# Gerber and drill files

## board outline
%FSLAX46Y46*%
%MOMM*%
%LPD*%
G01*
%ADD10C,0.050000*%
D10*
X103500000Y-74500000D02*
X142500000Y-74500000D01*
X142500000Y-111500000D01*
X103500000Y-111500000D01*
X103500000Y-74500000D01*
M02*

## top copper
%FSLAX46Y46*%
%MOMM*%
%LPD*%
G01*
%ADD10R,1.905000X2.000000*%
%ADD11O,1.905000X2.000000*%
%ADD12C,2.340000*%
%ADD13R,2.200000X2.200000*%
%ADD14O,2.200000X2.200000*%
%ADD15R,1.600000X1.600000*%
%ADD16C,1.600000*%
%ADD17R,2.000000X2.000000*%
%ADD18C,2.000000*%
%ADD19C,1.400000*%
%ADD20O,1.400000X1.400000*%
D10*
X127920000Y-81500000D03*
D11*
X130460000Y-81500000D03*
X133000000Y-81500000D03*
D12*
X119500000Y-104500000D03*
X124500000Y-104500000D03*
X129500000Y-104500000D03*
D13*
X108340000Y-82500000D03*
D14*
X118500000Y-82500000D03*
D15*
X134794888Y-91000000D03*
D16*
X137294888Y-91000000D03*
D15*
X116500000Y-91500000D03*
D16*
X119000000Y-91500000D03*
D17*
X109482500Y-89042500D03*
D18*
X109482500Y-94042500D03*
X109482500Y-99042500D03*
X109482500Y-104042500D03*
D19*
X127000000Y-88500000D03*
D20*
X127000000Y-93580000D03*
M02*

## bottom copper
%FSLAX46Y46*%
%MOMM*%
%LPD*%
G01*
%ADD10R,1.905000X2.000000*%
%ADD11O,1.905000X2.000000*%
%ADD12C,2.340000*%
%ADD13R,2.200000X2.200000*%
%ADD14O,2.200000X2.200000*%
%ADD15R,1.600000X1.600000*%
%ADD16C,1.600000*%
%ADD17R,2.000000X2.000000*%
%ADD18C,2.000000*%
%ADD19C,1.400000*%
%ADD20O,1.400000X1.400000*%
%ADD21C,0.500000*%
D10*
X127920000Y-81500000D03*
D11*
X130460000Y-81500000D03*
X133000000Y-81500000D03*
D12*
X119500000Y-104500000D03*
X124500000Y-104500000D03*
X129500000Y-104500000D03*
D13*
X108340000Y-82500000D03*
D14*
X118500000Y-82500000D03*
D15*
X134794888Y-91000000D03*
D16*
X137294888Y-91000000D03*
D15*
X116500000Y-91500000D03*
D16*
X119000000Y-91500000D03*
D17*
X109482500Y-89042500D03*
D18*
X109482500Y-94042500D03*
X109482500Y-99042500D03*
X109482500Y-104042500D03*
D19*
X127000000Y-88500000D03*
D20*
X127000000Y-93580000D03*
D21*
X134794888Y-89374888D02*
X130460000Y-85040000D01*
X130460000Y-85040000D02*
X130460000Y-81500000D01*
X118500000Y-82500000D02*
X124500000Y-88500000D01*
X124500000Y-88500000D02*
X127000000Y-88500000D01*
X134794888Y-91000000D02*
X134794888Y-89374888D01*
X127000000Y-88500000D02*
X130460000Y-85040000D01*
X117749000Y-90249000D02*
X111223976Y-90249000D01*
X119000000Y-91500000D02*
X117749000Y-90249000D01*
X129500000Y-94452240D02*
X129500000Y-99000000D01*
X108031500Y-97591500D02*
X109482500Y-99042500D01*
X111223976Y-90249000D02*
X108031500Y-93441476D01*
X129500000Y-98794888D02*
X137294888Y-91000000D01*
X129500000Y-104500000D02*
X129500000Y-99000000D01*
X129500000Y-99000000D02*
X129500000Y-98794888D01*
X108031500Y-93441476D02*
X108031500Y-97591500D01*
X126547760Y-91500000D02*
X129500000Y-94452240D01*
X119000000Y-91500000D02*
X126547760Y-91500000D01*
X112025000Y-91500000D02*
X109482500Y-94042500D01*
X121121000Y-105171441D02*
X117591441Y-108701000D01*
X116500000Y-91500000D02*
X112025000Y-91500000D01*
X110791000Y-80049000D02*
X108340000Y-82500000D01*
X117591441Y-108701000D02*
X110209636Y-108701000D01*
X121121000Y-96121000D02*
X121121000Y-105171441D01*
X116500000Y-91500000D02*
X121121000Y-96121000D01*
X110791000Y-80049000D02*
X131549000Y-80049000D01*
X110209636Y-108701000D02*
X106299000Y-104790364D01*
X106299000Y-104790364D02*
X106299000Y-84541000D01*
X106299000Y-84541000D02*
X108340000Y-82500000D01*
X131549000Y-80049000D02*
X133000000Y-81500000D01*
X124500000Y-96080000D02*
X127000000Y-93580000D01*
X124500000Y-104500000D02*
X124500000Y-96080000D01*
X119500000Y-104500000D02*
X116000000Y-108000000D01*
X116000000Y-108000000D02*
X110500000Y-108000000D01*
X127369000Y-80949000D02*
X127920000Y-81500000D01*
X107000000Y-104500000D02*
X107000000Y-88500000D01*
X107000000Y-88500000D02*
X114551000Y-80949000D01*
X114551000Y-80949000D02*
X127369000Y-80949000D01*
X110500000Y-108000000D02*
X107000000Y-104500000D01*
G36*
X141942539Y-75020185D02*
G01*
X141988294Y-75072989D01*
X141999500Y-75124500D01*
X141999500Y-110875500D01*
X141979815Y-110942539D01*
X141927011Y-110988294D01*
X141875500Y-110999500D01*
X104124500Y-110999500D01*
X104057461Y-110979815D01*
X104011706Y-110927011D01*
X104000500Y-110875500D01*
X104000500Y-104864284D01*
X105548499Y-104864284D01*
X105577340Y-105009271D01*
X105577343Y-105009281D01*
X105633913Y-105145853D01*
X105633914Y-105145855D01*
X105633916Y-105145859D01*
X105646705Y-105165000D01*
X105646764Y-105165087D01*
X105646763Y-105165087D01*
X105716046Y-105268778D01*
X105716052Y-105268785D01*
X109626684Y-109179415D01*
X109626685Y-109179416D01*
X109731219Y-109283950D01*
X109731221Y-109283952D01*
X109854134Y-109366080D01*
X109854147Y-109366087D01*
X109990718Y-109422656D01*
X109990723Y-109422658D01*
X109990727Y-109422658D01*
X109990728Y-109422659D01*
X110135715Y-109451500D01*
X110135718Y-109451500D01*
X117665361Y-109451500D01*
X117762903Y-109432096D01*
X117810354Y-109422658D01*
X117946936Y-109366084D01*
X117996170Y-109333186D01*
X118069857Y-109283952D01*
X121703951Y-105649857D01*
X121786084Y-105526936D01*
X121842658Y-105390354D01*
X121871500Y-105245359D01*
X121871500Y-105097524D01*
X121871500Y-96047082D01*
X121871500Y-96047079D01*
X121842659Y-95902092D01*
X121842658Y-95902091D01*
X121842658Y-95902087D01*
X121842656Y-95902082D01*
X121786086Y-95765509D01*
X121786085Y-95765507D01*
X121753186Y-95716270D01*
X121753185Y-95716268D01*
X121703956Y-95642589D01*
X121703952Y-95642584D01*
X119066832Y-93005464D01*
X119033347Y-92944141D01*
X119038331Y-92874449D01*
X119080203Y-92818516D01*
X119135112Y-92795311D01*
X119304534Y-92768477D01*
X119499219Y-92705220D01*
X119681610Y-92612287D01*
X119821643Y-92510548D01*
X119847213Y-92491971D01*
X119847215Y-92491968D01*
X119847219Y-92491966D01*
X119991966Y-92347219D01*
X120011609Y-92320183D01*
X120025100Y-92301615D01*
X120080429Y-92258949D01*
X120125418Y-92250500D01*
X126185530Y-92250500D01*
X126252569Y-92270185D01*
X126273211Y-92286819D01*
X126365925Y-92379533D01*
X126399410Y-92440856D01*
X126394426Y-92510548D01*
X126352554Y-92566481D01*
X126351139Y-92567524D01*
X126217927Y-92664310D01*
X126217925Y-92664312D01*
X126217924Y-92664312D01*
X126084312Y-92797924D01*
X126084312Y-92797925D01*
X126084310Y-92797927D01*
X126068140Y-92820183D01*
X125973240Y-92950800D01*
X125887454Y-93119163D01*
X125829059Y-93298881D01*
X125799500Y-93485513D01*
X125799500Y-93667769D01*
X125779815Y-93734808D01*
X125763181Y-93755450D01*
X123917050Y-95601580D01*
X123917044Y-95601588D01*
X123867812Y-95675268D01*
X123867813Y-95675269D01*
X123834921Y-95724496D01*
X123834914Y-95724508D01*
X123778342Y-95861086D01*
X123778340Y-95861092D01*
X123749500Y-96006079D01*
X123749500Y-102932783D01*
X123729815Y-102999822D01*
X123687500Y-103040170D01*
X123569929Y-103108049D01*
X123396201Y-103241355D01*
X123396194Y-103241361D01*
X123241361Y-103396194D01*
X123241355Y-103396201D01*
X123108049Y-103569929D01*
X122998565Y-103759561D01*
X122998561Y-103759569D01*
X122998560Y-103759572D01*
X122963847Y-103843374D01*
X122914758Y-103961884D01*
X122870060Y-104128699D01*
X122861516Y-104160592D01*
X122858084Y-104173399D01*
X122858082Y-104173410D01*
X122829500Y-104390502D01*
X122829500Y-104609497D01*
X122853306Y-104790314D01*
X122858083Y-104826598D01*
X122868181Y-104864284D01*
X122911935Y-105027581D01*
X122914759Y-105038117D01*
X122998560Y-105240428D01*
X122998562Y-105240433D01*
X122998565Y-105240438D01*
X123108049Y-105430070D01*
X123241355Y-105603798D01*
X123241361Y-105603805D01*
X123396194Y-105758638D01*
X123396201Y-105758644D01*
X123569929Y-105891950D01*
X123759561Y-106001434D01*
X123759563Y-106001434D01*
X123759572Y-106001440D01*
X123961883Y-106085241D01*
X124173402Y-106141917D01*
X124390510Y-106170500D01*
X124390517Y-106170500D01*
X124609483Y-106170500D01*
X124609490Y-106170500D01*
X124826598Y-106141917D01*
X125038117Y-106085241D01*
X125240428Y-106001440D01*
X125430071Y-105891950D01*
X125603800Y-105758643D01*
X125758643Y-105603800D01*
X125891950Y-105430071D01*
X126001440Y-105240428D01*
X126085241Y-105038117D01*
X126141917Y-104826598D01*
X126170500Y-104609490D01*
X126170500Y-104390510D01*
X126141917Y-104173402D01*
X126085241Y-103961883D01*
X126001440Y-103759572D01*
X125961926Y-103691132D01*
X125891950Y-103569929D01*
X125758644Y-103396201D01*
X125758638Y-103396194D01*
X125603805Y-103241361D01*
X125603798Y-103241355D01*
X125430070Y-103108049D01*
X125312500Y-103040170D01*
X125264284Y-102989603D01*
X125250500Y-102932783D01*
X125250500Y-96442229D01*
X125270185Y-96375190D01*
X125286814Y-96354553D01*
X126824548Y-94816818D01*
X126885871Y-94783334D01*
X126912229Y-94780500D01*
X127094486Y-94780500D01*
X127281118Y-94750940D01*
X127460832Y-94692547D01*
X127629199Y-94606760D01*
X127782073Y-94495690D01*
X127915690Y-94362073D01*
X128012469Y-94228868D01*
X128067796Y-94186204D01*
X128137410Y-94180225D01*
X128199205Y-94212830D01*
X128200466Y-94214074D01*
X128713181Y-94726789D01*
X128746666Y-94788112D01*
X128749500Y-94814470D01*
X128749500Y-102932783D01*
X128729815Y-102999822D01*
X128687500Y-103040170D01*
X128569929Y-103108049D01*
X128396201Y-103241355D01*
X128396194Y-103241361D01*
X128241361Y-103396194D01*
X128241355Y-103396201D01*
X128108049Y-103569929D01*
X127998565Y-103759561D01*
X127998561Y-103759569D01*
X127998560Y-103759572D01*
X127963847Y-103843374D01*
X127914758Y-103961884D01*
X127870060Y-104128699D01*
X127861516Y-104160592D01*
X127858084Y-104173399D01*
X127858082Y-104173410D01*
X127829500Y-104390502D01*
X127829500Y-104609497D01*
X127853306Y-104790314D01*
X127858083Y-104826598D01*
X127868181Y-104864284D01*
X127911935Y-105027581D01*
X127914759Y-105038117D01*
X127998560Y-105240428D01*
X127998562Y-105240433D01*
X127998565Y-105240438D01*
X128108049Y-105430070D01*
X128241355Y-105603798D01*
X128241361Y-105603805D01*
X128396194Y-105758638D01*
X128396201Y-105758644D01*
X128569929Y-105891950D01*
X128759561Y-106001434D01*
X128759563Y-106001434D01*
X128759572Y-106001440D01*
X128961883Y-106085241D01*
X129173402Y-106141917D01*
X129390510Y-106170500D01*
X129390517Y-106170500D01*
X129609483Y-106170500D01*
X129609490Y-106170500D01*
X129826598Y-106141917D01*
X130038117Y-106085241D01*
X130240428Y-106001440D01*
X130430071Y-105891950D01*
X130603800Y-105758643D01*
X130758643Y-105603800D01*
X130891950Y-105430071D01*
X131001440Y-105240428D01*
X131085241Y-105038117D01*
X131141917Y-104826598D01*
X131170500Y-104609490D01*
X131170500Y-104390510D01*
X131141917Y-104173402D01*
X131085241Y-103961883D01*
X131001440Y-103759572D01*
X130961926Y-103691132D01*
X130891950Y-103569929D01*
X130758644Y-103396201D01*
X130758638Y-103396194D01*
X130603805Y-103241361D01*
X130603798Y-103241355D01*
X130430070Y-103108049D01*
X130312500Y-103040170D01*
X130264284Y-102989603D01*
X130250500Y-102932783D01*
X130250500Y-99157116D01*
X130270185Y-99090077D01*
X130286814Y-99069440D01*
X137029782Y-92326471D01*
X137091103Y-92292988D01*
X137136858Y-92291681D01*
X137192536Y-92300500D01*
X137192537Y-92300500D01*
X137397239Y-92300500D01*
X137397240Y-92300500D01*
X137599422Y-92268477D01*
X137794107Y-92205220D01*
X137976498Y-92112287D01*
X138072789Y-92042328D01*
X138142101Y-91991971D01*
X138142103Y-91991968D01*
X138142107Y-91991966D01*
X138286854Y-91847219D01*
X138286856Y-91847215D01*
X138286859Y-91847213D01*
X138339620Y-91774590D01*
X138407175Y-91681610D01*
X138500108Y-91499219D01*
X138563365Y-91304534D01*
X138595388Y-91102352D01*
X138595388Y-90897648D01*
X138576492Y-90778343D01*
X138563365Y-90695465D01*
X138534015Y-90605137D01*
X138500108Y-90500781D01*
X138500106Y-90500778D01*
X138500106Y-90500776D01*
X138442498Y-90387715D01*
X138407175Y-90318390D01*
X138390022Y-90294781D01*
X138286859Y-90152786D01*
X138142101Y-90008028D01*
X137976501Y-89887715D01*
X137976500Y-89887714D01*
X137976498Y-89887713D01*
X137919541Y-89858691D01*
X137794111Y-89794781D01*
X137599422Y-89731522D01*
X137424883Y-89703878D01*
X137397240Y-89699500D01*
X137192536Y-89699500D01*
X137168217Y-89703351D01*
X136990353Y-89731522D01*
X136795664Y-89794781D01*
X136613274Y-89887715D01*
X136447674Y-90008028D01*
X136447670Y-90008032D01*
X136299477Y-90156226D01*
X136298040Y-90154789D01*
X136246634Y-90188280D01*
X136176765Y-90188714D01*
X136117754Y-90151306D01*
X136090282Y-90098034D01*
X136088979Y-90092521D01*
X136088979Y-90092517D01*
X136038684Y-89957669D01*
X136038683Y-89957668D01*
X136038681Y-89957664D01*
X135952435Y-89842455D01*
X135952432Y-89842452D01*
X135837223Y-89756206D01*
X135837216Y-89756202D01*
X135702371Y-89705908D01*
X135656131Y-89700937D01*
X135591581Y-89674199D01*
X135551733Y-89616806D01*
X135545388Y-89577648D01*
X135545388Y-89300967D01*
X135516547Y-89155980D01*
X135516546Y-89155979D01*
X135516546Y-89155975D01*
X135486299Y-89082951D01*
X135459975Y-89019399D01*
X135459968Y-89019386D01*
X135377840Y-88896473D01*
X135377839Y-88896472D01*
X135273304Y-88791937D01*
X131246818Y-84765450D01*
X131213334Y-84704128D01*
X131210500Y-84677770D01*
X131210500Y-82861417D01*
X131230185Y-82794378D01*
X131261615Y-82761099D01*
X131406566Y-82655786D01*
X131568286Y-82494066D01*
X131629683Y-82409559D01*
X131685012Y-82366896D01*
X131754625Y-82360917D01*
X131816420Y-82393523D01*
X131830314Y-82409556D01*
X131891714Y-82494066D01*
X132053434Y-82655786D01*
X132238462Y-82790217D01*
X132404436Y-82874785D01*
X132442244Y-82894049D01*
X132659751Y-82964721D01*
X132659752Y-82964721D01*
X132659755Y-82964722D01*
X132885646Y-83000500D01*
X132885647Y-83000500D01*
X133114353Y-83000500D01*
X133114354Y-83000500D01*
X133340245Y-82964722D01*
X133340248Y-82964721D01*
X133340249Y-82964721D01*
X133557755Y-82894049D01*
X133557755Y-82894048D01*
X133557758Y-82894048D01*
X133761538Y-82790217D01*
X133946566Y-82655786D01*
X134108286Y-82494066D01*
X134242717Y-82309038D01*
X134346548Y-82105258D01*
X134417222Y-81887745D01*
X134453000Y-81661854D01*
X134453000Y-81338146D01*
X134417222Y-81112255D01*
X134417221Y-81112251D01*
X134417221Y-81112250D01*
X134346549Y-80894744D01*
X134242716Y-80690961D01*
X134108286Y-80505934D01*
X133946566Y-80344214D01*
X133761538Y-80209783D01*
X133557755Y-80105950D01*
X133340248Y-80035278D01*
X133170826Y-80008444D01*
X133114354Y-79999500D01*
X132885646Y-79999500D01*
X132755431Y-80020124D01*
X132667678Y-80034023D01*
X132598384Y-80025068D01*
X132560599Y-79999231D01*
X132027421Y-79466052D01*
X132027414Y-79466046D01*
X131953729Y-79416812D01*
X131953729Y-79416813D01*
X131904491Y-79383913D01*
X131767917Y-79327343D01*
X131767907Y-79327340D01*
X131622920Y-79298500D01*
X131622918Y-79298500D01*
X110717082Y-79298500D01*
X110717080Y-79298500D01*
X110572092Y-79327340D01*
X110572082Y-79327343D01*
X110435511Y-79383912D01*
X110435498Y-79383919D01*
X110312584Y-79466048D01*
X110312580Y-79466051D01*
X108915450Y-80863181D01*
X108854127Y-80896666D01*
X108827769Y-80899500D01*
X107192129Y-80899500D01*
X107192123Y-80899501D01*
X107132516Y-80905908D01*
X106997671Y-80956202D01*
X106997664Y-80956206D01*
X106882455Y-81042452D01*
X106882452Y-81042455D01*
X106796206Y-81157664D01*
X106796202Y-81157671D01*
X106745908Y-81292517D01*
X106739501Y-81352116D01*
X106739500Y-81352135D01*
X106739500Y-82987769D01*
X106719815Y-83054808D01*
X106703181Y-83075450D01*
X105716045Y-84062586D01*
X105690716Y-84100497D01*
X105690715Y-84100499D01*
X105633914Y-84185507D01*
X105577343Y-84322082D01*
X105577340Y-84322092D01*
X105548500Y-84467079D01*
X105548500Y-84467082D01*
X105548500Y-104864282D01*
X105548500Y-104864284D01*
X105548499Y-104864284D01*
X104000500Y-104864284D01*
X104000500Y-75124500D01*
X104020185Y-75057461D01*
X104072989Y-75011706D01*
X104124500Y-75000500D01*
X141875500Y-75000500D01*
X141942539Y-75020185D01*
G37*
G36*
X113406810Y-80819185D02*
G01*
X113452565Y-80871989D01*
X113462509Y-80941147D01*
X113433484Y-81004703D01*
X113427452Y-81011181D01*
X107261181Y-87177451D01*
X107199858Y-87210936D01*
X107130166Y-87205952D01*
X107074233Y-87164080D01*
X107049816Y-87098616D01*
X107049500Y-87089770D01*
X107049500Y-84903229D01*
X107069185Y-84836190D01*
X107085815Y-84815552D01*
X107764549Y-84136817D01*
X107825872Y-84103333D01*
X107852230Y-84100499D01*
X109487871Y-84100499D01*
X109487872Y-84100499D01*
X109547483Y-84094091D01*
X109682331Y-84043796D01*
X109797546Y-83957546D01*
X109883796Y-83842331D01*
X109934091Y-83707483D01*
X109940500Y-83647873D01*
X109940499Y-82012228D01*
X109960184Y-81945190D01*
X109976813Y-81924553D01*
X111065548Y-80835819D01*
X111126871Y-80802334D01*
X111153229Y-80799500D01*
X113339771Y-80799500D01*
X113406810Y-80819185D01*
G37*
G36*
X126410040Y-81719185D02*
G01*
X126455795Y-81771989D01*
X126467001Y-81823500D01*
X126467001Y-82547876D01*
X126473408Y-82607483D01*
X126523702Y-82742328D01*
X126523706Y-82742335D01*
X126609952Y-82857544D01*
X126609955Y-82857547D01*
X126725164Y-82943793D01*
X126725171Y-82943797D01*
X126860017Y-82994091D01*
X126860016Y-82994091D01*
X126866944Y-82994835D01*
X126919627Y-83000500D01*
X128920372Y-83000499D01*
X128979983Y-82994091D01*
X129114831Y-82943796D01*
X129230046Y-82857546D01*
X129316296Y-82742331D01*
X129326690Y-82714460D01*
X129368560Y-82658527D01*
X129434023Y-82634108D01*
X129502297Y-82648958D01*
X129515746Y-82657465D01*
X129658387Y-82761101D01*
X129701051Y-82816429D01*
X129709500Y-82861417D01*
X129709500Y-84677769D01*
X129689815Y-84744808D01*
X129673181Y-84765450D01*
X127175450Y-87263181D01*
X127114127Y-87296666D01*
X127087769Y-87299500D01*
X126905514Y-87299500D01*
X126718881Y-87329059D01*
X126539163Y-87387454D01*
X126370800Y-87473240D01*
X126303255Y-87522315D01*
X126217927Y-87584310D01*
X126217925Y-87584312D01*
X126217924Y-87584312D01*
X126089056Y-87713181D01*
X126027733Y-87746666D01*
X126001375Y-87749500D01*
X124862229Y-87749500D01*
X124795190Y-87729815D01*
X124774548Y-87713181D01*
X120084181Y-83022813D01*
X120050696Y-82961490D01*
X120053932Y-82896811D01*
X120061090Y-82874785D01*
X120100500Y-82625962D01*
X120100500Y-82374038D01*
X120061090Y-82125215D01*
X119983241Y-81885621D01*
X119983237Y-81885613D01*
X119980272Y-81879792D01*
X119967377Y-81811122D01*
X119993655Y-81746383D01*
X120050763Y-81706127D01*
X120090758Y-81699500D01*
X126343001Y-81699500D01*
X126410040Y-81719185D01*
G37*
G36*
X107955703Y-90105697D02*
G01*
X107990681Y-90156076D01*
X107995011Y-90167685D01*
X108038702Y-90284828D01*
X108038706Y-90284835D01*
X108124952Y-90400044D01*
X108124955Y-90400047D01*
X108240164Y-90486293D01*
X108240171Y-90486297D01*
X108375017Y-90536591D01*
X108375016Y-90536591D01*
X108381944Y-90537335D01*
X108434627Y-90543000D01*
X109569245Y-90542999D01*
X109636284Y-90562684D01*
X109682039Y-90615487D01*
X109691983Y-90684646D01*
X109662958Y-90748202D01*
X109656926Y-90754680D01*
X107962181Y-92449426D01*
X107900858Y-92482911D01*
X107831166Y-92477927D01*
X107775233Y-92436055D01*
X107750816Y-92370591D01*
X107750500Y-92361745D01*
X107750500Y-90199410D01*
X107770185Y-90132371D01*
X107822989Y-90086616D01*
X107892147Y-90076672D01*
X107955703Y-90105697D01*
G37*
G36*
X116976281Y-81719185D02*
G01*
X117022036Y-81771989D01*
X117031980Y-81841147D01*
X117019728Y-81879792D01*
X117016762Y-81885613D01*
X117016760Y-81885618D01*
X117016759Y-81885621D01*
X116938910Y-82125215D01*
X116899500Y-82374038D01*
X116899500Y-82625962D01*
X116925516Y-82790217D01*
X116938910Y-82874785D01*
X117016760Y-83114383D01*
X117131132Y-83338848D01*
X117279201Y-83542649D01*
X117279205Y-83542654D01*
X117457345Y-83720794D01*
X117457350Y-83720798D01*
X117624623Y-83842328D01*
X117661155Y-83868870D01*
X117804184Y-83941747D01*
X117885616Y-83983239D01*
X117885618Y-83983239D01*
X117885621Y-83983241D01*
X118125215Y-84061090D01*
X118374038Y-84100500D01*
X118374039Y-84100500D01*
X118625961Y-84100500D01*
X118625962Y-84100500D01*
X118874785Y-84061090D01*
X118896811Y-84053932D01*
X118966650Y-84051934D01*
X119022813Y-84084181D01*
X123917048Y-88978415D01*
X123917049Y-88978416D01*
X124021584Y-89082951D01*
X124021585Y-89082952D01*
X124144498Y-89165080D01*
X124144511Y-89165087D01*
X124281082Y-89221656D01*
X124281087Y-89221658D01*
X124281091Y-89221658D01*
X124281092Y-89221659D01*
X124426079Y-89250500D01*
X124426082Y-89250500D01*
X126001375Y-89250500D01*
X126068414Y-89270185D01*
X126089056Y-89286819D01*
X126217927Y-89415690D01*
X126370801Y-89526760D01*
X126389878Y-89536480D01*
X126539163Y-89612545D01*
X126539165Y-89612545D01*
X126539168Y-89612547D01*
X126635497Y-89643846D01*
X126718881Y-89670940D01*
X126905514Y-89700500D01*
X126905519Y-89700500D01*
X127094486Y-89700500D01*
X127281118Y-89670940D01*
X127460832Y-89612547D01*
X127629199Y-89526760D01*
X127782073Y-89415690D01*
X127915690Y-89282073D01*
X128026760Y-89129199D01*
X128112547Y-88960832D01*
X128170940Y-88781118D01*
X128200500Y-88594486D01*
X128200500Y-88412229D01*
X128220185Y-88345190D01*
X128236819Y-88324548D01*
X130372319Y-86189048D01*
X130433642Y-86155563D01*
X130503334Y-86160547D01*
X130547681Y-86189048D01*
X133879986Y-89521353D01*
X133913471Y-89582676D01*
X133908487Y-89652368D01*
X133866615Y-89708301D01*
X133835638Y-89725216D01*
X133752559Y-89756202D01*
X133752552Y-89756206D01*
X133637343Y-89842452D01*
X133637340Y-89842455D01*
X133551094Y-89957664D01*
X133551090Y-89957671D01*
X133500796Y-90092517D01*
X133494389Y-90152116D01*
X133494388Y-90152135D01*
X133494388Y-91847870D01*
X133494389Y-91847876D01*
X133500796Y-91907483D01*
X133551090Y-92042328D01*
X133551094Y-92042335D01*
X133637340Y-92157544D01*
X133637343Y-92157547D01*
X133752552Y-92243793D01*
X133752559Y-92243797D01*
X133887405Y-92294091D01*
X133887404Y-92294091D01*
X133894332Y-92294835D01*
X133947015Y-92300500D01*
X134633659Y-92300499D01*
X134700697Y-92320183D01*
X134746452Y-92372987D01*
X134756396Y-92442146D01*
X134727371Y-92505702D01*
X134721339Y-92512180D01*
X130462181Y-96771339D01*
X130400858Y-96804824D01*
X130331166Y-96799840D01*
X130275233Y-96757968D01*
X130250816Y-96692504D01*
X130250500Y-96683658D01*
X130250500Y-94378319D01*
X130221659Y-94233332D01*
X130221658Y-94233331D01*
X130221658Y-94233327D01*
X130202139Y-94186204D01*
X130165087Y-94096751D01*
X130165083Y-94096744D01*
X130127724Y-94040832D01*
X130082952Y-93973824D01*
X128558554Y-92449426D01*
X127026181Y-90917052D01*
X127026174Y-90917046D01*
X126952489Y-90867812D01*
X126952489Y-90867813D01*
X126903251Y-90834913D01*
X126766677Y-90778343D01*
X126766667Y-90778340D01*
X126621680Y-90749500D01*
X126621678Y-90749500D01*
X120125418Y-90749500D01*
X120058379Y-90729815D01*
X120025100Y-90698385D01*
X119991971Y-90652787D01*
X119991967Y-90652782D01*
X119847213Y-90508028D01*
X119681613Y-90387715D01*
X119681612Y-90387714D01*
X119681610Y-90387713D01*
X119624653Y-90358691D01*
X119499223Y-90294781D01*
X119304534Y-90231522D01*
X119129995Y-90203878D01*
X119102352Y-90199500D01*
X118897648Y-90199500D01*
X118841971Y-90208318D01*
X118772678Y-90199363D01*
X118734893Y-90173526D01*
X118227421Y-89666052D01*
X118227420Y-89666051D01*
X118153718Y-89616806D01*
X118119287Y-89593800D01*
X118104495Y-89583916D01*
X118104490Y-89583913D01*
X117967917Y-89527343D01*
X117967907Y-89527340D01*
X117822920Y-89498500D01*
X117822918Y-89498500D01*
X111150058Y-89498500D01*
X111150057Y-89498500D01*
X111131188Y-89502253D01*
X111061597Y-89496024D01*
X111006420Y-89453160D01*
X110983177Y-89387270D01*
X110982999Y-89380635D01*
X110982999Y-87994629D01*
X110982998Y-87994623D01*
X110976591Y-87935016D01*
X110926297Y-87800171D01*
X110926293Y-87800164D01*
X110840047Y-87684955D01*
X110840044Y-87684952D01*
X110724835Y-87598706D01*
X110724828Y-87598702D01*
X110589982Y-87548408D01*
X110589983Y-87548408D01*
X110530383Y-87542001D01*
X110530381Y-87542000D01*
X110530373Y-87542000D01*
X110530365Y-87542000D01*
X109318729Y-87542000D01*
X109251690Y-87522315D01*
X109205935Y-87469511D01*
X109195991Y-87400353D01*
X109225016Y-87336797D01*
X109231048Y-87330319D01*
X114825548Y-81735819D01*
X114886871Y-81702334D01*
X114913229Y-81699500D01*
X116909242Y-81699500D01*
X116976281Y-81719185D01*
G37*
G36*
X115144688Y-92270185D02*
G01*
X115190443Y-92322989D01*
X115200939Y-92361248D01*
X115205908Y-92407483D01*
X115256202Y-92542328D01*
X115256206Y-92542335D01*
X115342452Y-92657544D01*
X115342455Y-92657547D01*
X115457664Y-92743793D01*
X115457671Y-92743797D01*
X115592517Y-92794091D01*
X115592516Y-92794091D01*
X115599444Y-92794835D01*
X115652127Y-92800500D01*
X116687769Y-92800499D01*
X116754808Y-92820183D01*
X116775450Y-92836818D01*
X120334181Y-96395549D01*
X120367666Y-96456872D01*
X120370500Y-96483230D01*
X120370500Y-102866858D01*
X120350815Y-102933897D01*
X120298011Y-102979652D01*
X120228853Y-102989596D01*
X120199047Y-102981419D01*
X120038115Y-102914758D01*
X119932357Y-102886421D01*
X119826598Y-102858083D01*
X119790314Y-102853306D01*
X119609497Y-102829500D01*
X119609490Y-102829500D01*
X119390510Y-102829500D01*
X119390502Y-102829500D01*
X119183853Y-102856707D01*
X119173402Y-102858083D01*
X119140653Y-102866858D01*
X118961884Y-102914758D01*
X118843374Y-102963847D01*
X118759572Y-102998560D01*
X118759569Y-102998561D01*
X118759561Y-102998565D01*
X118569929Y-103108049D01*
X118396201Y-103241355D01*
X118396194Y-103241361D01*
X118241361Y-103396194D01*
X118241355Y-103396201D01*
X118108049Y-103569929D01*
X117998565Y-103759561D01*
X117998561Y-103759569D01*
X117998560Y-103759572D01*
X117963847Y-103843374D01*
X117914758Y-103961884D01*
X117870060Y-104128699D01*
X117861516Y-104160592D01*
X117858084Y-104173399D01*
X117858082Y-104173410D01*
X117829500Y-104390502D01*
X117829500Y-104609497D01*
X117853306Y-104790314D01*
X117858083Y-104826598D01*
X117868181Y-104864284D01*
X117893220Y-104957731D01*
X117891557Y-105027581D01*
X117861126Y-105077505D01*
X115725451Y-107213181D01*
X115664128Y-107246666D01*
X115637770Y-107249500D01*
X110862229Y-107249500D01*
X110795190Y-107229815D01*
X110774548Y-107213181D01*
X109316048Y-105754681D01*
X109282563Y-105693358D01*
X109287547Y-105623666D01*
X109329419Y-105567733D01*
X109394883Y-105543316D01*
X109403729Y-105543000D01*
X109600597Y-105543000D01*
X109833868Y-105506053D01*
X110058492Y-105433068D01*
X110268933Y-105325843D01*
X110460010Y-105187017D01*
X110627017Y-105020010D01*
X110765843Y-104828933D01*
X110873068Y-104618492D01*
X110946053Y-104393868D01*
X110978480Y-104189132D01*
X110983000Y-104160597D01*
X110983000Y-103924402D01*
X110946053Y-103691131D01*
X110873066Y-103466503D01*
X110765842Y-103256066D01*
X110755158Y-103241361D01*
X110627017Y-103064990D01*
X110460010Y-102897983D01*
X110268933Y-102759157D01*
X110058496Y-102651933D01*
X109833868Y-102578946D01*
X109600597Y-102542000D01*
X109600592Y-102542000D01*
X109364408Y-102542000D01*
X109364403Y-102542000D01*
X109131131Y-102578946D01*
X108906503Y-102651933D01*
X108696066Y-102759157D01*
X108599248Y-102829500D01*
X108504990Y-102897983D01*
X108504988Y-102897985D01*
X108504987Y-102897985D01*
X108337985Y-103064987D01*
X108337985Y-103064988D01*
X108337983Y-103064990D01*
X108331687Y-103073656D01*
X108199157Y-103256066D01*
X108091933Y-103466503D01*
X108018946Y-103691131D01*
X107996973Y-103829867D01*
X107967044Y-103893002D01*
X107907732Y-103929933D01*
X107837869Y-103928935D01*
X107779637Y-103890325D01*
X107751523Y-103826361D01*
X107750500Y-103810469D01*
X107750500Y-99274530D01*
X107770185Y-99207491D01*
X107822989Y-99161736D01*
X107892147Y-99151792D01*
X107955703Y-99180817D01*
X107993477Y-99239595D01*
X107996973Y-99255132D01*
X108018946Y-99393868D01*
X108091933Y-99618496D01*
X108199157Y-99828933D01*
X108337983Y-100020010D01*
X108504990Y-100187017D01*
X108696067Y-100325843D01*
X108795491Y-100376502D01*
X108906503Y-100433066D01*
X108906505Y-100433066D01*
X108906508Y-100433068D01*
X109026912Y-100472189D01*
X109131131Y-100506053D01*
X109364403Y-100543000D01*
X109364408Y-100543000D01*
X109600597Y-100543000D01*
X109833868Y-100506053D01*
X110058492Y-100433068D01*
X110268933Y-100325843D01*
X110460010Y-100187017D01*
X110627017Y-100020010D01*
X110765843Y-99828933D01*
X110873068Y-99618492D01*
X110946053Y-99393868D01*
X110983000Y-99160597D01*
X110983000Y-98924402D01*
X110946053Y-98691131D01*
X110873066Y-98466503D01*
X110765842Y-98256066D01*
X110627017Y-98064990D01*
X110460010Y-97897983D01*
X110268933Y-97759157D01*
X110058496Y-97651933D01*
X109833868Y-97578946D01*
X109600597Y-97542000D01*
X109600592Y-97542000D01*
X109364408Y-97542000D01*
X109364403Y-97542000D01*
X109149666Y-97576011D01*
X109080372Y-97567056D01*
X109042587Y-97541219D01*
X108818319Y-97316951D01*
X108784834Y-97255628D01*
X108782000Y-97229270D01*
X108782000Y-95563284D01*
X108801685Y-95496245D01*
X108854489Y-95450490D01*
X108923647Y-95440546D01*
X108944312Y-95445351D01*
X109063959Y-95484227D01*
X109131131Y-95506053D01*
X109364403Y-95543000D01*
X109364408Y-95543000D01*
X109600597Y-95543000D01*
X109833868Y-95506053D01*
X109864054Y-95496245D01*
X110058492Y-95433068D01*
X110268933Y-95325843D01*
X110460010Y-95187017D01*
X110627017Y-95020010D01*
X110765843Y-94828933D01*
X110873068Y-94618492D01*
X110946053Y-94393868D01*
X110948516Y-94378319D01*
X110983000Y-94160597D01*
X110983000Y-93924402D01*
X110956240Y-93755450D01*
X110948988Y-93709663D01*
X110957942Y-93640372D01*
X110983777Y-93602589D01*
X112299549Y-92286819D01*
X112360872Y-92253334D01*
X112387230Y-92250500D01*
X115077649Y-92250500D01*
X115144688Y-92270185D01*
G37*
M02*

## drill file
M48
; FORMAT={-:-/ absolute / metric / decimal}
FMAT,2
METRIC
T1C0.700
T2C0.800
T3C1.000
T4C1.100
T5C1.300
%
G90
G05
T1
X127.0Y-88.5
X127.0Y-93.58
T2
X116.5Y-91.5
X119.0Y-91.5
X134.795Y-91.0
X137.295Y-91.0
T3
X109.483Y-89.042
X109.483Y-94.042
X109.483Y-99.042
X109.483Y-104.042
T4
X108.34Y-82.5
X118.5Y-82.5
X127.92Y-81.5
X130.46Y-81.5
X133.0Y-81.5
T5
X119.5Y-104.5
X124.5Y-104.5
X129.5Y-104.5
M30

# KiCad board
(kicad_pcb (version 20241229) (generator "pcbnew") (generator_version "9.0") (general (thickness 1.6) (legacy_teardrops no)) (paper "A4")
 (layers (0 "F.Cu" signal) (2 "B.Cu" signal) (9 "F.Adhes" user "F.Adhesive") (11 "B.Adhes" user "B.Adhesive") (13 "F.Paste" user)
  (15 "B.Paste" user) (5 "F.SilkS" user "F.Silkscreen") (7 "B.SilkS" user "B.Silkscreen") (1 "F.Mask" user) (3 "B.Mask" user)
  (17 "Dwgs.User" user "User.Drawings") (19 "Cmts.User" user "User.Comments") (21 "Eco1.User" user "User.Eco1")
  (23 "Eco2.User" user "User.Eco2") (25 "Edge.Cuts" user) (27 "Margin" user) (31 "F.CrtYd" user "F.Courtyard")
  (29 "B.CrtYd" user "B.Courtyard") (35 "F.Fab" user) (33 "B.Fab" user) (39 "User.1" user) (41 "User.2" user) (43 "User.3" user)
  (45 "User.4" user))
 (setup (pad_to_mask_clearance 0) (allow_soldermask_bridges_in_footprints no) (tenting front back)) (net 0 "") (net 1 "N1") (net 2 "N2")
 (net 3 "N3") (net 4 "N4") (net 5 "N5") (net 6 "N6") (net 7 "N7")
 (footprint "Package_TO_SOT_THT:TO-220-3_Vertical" (layer "F.Cu") (at 127.92 81.5)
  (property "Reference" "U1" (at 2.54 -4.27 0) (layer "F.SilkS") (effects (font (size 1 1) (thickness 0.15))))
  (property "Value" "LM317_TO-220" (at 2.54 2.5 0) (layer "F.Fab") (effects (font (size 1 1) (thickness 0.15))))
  (pad "1" thru_hole rect (at 0 0) (size 1.905 2) (drill 1.1) (layers "*.Cu" "*.Mask") (remove_unused_layers no) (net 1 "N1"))
  (pad "2" thru_hole oval (at 2.54 0) (size 1.905 2) (drill 1.1) (layers "*.Cu" "*.Mask") (remove_unused_layers no) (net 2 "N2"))
  (pad "3" thru_hole oval (at 5.08 0) (size 1.905 2) (drill 1.1) (layers "*.Cu" "*.Mask") (remove_unused_layers no) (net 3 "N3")))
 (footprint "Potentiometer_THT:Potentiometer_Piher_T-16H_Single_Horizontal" (layer "F.Cu") (at 119.5 104.5 -90)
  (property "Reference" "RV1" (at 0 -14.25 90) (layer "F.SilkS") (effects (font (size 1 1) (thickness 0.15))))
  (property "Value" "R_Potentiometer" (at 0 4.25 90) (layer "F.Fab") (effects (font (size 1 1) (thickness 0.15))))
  (pad "1" thru_hole circle (at 0 0 270) (size 2.34 2.34) (drill 1.3) (layers "*.Cu" "*.Mask") (remove_unused_layers no) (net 1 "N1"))
  (pad "2" thru_hole circle (at 0 -5 270) (size 2.34 2.34) (drill 1.3) (layers "*.Cu" "*.Mask") (remove_unused_layers no) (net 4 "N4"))
  (pad "3" thru_hole circle (at 0 -10 270) (size 2.34 2.34) (drill 1.3) (layers "*.Cu" "*.Mask") (remove_unused_layers no) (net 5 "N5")))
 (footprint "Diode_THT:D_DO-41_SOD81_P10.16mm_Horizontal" (layer "F.Cu") (at 108.34 82.5)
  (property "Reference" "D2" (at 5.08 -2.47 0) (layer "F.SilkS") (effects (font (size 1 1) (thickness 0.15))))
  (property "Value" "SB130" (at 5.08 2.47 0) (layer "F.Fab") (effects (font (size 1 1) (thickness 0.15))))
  (pad "1" thru_hole rect (at 0 0) (size 2.2 2.2) (drill 1.1) (layers "*.Cu" "*.Mask") (remove_unused_layers no) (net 3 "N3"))
  (pad "2" thru_hole oval (at 10.16 0) (size 2.2 2.2) (drill 1.1) (layers "*.Cu" "*.Mask") (remove_unused_layers no) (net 2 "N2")))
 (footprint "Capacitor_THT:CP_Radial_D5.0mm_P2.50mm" (layer "F.Cu") (at 134.794888 91)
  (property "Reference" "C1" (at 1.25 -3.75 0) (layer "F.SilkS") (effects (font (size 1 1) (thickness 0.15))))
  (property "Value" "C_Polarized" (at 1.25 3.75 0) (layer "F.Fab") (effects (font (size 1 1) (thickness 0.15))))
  (pad "1" thru_hole rect (at 0 0) (size 1.6 1.6) (drill 0.8) (layers "*.Cu" "*.Mask") (remove_unused_layers no) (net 2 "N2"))
  (pad "2" thru_hole circle (at 2.5 0) (size 1.6 1.6) (drill 0.8) (layers "*.Cu" "*.Mask") (remove_unused_layers no) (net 5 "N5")))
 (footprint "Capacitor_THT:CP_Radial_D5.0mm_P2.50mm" (layer "F.Cu") (at 116.5 91.5)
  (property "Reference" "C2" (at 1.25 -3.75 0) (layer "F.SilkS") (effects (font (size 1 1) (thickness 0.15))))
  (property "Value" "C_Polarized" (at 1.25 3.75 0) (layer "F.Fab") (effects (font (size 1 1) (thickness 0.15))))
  (pad "1" thru_hole rect (at 0 0) (size 1.6 1.6) (drill 0.8) (layers "*.Cu" "*.Mask") (remove_unused_layers no) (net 3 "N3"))
  (pad "2" thru_hole circle (at 2.5 0) (size 1.6 1.6) (drill 0.8) (layers "*.Cu" "*.Mask") (remove_unused_layers no) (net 5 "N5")))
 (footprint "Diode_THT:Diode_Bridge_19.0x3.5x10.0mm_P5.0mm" (layer "F.Cu") (at 109.4825 89.0425 -90)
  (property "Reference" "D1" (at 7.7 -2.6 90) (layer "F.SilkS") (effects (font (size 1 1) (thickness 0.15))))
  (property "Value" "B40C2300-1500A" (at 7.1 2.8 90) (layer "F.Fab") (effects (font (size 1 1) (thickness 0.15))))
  (pad "1" thru_hole rect (at 0 0 270) (size 2 2) (drill 1) (layers "*.Cu" "*.Mask") (remove_unused_layers no) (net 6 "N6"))
  (pad "2" thru_hole circle (at 5 0 270) (size 2 2) (drill 1) (layers "*.Cu" "*.Mask") (remove_unused_layers no) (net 3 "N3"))
  (pad "3" thru_hole circle (at 10 0 270) (size 2 2) (drill 1) (layers "*.Cu" "*.Mask") (remove_unused_layers no) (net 5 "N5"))
  (pad "4" thru_hole circle (at 15 0 270) (size 2 2) (drill 1) (layers "*.Cu" "*.Mask") (remove_unused_layers no) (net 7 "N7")))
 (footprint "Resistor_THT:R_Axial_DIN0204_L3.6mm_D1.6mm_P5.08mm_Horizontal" (layer "F.Cu") (at 127 88.5 -90)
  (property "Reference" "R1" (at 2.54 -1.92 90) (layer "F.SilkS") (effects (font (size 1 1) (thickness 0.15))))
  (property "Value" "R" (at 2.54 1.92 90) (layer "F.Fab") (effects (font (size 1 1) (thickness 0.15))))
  (pad "1" thru_hole circle (at 0 0 270) (size 1.4 1.4) (drill 0.7) (layers "*.Cu" "*.Mask") (remove_unused_layers no) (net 2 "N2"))
  (pad "2" thru_hole oval (at 5.08 0 270) (size 1.4 1.4) (drill 0.7) (layers "*.Cu" "*.Mask") (remove_unused_layers no) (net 4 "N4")))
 (gr_rect (start 103.5 74.5) (end 142.5 111.5) (stroke (width 0.05) (type default)) (fill no) (layer "Edge.Cuts"))
 (segment (start 134.794888 89.374888) (end 130.46 85.04) (width 0.5) (layer "B.Cu") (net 2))
 (segment (start 130.46 85.04) (end 130.46 81.5) (width 0.5) (layer "B.Cu") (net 2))
 (segment (start 118.5 82.5) (end 124.5 88.5) (width 0.5) (layer "B.Cu") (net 2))
 (segment (start 124.5 88.5) (end 127 88.5) (width 0.5) (layer "B.Cu") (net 2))
 (segment (start 134.794888 91) (end 134.794888 89.374888) (width 0.5) (layer "B.Cu") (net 2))
 (segment (start 127 88.5) (end 130.46 85.04) (width 0.5) (layer "B.Cu") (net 2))
 (segment (start 117.749 90.249) (end 111.223976 90.249) (width 0.5) (layer "B.Cu") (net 5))
 (segment (start 119 91.5) (end 117.749 90.249) (width 0.5) (layer "B.Cu") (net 5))
 (segment (start 129.5 94.45224) (end 129.5 99) (width 0.5) (layer "B.Cu") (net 5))
 (segment (start 108.0315 97.5915) (end 109.4825 99.0425) (width 0.5) (layer "B.Cu") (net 5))
 (segment (start 111.223976 90.249) (end 108.0315 93.441476) (width 0.5) (layer "B.Cu") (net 5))
 (segment (start 129.5 98.794888) (end 137.294888 91) (width 0.5) (layer "B.Cu") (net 5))
 (segment (start 129.5 104.5) (end 129.5 99) (width 0.5) (layer "B.Cu") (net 5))
 (segment (start 129.5 99) (end 129.5 98.794888) (width 0.5) (layer "B.Cu") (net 5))
 (segment (start 108.0315 93.441476) (end 108.0315 97.5915) (width 0.5) (layer "B.Cu") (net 5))
 (segment (start 126.54776 91.5) (end 129.5 94.45224) (width 0.5) (layer "B.Cu") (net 5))
 (segment (start 119 91.5) (end 126.54776 91.5) (width 0.5) (layer "B.Cu") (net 5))
 (segment (start 112.025 91.5) (end 109.4825 94.0425) (width 0.5) (layer "B.Cu") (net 3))
 (segment (start 121.121 105.171441) (end 117.591441 108.701) (width 0.5) (layer "B.Cu") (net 3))
 (segment (start 116.5 91.5) (end 112.025 91.5) (width 0.5) (layer "B.Cu") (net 3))
 (segment (start 110.791 80.049) (end 108.34 82.5) (width 0.5) (layer "B.Cu") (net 3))
 (segment (start 117.591441 108.701) (end 110.209636 108.701) (width 0.5) (layer "B.Cu") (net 3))
 (segment (start 121.121 96.121) (end 121.121 105.171441) (width 0.5) (layer "B.Cu") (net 3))
 (segment (start 116.5 91.5) (end 121.121 96.121) (width 0.5) (layer "B.Cu") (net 3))
 (segment (start 110.791 80.049) (end 131.549 80.049) (width 0.5) (layer "B.Cu") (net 3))
 (segment (start 110.209636 108.701) (end 106.299 104.790364) (width 0.5) (layer "B.Cu") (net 3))
 (segment (start 106.299 104.790364) (end 106.299 84.541) (width 0.5) (layer "B.Cu") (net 3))
 (segment (start 106.299 84.541) (end 108.34 82.5) (width 0.5) (layer "B.Cu") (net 3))
 (segment (start 131.549 80.049) (end 133 81.5) (width 0.5) (layer "B.Cu") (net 3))
 (segment (start 124.5 96.08) (end 127 93.58) (width 0.5) (layer "B.Cu") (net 4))
 (segment (start 124.5 104.5) (end 124.5 96.08) (width 0.5) (layer "B.Cu") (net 4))
 (segment (start 119.5 104.5) (end 116 108) (width 0.5) (layer "B.Cu") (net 1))
 (segment (start 116 108) (end 110.5 108) (width 0.5) (layer "B.Cu") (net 1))
 (segment (start 127.369 80.949) (end 127.92 81.5) (width 0.5) (layer "B.Cu") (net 1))
 (segment (start 107 104.5) (end 107 88.5) (width 0.5) (layer "B.Cu") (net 1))
 (segment (start 107 88.5) (end 114.551 80.949) (width 0.5) (layer "B.Cu") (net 1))
 (segment (start 114.551 80.949) (end 127.369 80.949) (width 0.5) (layer "B.Cu") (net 1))
 (segment (start 110.5 108) (end 107 104.5) (width 0.5) (layer "B.Cu") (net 1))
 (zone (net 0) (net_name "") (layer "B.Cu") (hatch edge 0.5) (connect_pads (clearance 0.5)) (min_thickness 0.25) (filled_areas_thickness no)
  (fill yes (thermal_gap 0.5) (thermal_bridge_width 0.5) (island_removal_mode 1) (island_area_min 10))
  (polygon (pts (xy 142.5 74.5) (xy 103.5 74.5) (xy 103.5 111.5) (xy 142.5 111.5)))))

